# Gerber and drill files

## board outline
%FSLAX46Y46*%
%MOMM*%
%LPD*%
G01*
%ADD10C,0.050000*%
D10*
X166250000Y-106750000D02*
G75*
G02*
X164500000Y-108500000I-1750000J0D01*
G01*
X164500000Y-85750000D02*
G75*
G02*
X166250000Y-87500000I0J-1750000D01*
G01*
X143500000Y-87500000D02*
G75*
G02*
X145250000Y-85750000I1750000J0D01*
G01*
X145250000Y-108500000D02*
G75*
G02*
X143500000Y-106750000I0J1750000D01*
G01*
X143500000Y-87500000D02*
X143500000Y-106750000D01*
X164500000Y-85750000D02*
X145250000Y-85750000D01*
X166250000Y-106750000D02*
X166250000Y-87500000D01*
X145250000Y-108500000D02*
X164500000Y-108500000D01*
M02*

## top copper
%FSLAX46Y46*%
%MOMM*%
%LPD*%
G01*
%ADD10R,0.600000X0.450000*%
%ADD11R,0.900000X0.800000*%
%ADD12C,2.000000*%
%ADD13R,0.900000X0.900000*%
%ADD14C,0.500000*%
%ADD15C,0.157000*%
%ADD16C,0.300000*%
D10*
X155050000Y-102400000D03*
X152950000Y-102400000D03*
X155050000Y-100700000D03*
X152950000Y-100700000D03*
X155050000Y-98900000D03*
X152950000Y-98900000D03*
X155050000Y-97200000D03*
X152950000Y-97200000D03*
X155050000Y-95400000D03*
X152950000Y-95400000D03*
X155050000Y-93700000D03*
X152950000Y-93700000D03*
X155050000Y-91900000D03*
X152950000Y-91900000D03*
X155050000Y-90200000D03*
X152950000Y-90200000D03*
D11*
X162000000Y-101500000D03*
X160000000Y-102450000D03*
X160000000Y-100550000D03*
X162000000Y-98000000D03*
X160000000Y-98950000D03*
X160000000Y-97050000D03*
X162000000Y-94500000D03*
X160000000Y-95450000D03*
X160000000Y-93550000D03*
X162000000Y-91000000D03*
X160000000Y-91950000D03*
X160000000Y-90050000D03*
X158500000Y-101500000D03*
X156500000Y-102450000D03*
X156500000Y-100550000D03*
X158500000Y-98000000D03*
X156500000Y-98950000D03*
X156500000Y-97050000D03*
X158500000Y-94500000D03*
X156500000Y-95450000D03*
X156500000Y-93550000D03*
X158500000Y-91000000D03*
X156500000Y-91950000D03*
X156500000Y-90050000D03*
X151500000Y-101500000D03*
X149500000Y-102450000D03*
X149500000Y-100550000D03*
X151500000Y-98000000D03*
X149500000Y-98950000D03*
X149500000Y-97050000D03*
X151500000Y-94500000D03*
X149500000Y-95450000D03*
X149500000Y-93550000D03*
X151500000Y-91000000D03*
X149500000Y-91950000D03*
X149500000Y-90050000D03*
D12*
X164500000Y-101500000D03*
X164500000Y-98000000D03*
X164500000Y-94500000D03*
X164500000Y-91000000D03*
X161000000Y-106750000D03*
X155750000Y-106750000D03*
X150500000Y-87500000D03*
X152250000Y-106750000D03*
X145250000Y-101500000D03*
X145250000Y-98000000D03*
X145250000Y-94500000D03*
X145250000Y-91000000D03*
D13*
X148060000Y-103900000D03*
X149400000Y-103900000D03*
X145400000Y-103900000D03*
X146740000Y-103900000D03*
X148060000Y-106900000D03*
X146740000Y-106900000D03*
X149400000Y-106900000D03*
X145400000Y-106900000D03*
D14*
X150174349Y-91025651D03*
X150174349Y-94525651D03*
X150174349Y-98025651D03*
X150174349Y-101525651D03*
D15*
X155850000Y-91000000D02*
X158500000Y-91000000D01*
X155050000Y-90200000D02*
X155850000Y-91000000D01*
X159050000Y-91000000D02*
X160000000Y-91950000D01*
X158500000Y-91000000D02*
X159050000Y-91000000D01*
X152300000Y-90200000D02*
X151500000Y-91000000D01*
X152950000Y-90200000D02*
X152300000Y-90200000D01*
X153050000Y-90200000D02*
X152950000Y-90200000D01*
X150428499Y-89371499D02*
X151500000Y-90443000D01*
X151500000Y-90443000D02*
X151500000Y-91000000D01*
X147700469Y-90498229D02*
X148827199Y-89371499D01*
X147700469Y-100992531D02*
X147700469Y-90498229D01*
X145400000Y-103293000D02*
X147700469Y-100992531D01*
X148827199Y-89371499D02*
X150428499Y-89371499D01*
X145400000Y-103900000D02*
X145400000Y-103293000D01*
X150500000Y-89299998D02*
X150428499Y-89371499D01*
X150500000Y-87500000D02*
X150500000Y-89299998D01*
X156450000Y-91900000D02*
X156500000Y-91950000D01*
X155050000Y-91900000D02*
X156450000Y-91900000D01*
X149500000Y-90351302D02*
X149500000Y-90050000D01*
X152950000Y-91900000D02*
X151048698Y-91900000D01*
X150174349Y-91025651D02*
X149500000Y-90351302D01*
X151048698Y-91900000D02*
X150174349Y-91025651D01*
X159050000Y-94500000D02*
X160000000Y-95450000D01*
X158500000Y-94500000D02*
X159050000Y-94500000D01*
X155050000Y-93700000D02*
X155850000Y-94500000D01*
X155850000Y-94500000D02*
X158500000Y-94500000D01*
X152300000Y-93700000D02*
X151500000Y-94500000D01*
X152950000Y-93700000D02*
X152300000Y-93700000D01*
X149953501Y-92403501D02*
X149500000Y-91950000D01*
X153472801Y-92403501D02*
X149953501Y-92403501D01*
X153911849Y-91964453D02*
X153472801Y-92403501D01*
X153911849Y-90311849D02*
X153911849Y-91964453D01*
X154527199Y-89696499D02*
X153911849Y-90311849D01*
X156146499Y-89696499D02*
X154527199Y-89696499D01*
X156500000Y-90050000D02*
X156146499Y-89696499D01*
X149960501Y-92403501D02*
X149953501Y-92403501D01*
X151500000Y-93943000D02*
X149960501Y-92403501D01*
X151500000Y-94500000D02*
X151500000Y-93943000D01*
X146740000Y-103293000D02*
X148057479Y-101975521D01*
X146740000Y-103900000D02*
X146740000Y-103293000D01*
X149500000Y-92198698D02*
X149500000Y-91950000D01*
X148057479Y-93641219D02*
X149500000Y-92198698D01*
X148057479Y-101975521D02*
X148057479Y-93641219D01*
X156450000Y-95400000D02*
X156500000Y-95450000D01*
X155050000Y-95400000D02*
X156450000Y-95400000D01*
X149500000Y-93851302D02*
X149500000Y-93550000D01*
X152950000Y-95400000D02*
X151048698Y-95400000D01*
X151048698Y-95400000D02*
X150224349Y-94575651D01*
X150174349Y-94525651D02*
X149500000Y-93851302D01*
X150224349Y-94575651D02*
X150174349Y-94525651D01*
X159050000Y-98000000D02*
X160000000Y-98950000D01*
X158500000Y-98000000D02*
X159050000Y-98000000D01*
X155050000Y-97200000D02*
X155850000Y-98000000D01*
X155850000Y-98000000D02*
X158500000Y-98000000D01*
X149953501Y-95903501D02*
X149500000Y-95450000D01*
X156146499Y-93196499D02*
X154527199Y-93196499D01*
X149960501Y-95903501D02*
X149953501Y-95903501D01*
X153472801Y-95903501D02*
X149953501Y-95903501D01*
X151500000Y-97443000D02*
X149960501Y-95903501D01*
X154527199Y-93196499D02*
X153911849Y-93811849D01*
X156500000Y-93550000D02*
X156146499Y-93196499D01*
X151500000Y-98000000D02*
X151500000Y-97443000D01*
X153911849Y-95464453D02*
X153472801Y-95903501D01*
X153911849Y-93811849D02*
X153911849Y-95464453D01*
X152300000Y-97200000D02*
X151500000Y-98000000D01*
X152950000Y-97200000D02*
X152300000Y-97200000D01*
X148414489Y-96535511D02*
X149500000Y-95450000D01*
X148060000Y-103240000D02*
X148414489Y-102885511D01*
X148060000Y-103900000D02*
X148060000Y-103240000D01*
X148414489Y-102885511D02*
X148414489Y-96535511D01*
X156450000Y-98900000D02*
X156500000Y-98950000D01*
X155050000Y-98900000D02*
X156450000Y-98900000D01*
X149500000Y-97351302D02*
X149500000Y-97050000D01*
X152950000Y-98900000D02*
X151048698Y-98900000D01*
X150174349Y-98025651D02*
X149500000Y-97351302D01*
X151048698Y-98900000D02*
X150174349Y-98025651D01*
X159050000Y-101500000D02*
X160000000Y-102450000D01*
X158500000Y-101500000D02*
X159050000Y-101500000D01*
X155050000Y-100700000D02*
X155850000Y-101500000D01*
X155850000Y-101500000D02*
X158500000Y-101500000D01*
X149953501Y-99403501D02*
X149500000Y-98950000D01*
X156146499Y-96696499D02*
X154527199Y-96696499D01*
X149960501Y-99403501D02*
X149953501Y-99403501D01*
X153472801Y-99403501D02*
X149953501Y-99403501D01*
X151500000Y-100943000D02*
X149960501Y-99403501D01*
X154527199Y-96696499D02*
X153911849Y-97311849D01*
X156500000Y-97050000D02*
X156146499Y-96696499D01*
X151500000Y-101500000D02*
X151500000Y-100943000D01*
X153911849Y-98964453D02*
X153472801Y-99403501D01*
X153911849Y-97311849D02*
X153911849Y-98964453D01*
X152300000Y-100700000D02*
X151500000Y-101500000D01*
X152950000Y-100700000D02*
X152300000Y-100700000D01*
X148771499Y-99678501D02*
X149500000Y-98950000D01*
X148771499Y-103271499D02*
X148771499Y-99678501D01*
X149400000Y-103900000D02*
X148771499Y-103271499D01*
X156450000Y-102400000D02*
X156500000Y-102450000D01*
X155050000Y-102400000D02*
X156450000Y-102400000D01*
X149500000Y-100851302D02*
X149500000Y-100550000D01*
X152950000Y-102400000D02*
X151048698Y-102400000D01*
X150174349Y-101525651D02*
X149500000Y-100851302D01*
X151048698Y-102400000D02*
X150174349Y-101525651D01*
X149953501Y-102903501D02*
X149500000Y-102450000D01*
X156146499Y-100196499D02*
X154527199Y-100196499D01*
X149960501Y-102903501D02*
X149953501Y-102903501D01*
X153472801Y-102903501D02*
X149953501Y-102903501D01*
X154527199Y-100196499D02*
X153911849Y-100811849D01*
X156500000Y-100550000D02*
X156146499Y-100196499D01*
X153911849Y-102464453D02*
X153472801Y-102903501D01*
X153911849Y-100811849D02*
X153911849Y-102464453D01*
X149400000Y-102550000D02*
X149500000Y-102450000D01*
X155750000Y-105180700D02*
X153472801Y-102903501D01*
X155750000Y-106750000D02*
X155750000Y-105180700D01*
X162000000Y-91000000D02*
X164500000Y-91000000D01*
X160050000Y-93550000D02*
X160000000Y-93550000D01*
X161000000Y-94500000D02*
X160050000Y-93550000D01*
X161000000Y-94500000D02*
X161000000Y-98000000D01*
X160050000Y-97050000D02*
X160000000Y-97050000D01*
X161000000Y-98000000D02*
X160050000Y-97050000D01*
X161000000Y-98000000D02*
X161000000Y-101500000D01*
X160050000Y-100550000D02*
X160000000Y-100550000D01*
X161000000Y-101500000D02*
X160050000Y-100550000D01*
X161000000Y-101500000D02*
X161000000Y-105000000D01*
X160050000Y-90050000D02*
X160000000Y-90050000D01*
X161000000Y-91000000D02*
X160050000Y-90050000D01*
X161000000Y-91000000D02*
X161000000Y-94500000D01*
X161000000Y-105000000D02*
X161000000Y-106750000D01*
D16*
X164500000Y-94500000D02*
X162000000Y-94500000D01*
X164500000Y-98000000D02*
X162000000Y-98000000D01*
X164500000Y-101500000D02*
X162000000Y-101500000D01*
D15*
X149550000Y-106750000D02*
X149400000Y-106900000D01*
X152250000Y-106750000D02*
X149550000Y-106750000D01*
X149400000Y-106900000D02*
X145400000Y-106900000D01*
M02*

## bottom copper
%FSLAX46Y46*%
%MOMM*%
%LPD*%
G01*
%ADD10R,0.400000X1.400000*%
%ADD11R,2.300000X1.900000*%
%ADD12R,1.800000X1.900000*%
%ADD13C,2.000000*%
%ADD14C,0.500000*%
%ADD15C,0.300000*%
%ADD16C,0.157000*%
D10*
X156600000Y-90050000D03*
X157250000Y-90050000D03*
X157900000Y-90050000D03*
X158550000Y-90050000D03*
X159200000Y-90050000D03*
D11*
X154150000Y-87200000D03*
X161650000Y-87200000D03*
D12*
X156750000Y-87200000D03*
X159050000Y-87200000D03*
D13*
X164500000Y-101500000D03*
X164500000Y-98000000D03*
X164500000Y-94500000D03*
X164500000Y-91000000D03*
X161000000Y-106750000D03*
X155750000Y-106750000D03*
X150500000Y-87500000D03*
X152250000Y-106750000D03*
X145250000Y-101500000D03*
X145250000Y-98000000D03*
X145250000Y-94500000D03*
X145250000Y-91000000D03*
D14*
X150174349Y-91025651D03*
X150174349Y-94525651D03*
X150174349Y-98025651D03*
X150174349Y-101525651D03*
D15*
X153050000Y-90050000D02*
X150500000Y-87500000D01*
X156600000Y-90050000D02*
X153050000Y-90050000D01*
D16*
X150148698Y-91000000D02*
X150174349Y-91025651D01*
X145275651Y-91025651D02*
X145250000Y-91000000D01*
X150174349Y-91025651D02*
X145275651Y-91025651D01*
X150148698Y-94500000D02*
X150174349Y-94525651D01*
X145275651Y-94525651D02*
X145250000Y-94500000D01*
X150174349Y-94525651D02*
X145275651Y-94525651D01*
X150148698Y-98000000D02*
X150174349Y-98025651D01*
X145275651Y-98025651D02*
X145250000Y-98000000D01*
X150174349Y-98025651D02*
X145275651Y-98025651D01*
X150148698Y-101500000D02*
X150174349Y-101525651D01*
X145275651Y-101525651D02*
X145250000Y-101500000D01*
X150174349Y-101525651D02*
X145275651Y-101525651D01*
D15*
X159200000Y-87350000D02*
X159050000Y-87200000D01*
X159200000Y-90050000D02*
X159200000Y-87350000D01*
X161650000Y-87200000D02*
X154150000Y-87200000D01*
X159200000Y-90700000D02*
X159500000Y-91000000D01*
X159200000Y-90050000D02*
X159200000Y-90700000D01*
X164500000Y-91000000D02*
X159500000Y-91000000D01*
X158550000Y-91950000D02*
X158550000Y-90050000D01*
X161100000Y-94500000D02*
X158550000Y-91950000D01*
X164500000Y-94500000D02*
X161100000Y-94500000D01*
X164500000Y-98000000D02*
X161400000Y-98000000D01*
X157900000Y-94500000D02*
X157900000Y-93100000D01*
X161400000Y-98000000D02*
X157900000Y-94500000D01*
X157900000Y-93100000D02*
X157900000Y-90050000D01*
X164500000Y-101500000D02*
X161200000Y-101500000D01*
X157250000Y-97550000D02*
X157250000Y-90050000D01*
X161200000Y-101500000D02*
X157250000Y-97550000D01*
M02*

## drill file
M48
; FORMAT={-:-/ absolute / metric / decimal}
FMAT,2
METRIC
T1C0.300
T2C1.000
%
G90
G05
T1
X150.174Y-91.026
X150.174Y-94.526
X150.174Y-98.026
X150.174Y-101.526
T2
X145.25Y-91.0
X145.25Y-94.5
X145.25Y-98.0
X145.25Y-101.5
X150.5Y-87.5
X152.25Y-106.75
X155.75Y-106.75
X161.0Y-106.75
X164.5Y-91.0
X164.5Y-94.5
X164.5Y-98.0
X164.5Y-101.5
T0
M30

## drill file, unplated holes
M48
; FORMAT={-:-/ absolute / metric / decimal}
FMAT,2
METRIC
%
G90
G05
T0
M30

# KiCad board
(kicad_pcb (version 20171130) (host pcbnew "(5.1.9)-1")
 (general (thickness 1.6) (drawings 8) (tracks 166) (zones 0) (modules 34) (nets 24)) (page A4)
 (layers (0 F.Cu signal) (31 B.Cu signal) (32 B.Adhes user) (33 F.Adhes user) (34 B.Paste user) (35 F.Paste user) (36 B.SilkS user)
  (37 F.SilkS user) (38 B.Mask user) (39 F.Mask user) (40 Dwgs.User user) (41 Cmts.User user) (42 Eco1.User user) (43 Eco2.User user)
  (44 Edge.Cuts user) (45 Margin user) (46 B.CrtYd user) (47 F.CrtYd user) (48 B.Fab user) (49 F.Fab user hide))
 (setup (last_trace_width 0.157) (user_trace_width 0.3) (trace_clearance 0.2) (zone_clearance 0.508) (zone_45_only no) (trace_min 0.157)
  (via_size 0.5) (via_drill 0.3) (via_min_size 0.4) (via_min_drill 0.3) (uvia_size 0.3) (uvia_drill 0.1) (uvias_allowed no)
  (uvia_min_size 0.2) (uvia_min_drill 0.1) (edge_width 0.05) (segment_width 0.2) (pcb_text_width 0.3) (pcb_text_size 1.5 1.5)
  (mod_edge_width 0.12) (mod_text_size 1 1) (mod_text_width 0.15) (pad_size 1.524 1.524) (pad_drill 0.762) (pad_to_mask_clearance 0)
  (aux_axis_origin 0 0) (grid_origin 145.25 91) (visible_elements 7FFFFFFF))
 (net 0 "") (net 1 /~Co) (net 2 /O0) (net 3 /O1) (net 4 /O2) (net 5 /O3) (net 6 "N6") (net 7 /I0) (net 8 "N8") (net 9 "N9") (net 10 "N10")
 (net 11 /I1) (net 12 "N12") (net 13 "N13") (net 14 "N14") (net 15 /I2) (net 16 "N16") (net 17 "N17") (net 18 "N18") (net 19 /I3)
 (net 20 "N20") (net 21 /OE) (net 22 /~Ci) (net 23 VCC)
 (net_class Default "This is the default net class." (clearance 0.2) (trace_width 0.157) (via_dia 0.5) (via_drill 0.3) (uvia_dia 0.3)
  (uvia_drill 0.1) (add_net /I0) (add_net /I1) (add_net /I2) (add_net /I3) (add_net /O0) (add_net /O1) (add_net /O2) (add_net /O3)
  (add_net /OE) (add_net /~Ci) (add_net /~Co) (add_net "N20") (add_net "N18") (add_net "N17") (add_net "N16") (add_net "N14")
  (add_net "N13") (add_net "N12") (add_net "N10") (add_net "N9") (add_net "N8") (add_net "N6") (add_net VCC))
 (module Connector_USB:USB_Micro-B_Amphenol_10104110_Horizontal (layer B.Cu) (at 157.9 88.5)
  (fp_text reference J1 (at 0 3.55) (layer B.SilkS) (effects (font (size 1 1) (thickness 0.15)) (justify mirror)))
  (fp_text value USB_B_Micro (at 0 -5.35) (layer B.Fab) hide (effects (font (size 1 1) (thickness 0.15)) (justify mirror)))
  (pad 1 smd rect (at -1.3 1.55) (size 0.4 1.4) (layers B.Cu B.Paste B.Mask) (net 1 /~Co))
  (pad 2 smd rect (at -0.65 1.55) (size 0.4 1.4) (layers B.Cu B.Paste B.Mask) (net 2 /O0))
  (pad 3 smd rect (at 0 1.55) (size 0.4 1.4) (layers B.Cu B.Paste B.Mask) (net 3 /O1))
  (pad 4 smd rect (at 0.65 1.55) (size 0.4 1.4) (layers B.Cu B.Paste B.Mask) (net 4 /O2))
  (pad 5 smd rect (at 1.3 1.55) (size 0.4 1.4) (layers B.Cu B.Paste B.Mask) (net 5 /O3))
  (pad 6 smd rect (at -3.75 -1.3) (size 2.3 1.9) (layers B.Cu B.Paste B.Mask) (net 5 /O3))
  (pad 6 smd rect (at 3.75 -1.3) (size 2.3 1.9) (layers B.Cu B.Paste B.Mask) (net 5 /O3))
  (pad 6 smd rect (at -1.15 -1.3) (size 1.8 1.9) (layers B.Cu B.Paste B.Mask) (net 5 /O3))
  (pad 6 smd rect (at 1.15 -1.3) (size 1.8 1.9) (layers B.Cu B.Paste B.Mask) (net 5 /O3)))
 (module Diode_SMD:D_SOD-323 (layer F.Cu) (at 154 102.4)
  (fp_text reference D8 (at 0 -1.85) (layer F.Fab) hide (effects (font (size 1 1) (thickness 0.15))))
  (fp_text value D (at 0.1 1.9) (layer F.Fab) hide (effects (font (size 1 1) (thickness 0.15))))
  (pad 2 smd rect (at 1.05 0) (size 0.6 0.45) (layers F.Cu F.Paste F.Mask) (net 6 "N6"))
  (pad 1 smd rect (at -1.05 0) (size 0.6 0.45) (layers F.Cu F.Paste F.Mask) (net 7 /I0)))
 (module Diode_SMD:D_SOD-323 (layer F.Cu) (at 154 100.7)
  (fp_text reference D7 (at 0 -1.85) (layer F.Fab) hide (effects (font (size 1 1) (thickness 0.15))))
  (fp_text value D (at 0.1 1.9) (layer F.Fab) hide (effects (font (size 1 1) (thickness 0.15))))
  (pad 2 smd rect (at 1.05 0) (size 0.6 0.45) (layers F.Cu F.Paste F.Mask) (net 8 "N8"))
  (pad 1 smd rect (at -1.05 0) (size 0.6 0.45) (layers F.Cu F.Paste F.Mask) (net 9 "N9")))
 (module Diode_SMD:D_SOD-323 (layer F.Cu) (at 154 98.9)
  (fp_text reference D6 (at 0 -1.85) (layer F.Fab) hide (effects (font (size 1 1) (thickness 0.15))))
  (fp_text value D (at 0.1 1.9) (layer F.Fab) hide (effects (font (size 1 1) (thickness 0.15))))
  (pad 2 smd rect (at 1.05 0) (size 0.6 0.45) (layers F.Cu F.Paste F.Mask) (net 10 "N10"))
  (pad 1 smd rect (at -1.05 0) (size 0.6 0.45) (layers F.Cu F.Paste F.Mask) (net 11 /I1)))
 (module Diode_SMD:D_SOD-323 (layer F.Cu) (at 154 97.2)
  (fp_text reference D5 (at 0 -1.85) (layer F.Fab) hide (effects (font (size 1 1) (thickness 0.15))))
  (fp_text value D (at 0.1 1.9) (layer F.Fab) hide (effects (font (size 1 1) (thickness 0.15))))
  (pad 2 smd rect (at 1.05 0) (size 0.6 0.45) (layers F.Cu F.Paste F.Mask) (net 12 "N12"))
  (pad 1 smd rect (at -1.05 0) (size 0.6 0.45) (layers F.Cu F.Paste F.Mask) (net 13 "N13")))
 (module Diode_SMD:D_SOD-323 (layer F.Cu) (at 154 95.4)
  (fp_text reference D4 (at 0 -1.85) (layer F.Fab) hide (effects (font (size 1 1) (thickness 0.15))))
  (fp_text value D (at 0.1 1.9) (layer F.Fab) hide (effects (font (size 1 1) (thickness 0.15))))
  (pad 2 smd rect (at 1.05 0) (size 0.6 0.45) (layers F.Cu F.Paste F.Mask) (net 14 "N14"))
  (pad 1 smd rect (at -1.05 0) (size 0.6 0.45) (layers F.Cu F.Paste F.Mask) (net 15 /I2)))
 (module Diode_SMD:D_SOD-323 (layer F.Cu) (at 154 93.7)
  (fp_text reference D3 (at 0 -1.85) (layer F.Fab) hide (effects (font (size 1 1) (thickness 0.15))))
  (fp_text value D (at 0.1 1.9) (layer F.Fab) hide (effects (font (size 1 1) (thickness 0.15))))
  (pad 2 smd rect (at 1.05 0) (size 0.6 0.45) (layers F.Cu F.Paste F.Mask) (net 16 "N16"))
  (pad 1 smd rect (at -1.05 0) (size 0.6 0.45) (layers F.Cu F.Paste F.Mask) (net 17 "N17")))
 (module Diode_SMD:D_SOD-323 (layer F.Cu) (at 154 91.9)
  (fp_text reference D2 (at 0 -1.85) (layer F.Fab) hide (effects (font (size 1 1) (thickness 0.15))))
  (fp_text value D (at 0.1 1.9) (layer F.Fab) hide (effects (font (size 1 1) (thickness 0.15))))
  (pad 2 smd rect (at 1.05 0) (size 0.6 0.45) (layers F.Cu F.Paste F.Mask) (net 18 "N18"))
  (pad 1 smd rect (at -1.05 0) (size 0.6 0.45) (layers F.Cu F.Paste F.Mask) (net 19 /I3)))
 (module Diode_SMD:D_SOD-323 (layer F.Cu) (at 154 90.2)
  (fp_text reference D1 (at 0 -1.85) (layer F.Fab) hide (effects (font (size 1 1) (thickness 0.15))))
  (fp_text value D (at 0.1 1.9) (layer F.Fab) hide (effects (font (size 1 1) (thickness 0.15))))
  (pad 2 smd rect (at 1.05 0) (size 0.6 0.45) (layers F.Cu F.Paste F.Mask) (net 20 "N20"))
  (pad 1 smd rect (at -1.05 0) (size 0.6 0.45) (layers F.Cu F.Paste F.Mask) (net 1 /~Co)))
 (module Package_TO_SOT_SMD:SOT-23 (layer F.Cu) (at 161 101.5)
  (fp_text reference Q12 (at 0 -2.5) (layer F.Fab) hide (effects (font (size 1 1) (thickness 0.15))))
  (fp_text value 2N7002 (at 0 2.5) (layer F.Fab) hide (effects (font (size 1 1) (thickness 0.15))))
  (pad 3 smd rect (at 1 0) (size 0.9 0.8) (layers F.Cu F.Paste F.Mask) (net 2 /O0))
  (pad 2 smd rect (at -1 0.95) (size 0.9 0.8) (layers F.Cu F.Paste F.Mask) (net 8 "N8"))
  (pad 1 smd rect (at -1 -0.95) (size 0.9 0.8) (layers F.Cu F.Paste F.Mask) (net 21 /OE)))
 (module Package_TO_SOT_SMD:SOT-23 (layer F.Cu) (at 161 98)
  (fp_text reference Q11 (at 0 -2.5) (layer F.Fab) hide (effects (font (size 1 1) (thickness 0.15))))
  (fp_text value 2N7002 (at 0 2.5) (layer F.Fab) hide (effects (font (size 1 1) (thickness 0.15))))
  (pad 3 smd rect (at 1 0) (size 0.9 0.8) (layers F.Cu F.Paste F.Mask) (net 3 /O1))
  (pad 2 smd rect (at -1 0.95) (size 0.9 0.8) (layers F.Cu F.Paste F.Mask) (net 12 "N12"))
  (pad 1 smd rect (at -1 -0.95) (size 0.9 0.8) (layers F.Cu F.Paste F.Mask) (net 21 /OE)))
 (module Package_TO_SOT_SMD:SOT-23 (layer F.Cu) (at 161 94.5)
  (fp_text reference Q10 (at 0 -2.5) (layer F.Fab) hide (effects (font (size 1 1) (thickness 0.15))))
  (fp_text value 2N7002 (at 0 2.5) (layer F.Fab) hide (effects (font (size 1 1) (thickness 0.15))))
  (pad 3 smd rect (at 1 0) (size 0.9 0.8) (layers F.Cu F.Paste F.Mask) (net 4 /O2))
  (pad 2 smd rect (at -1 0.95) (size 0.9 0.8) (layers F.Cu F.Paste F.Mask) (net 16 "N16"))
  (pad 1 smd rect (at -1 -0.95) (size 0.9 0.8) (layers F.Cu F.Paste F.Mask) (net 21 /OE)))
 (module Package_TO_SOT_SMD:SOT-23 (layer F.Cu) (at 161 91)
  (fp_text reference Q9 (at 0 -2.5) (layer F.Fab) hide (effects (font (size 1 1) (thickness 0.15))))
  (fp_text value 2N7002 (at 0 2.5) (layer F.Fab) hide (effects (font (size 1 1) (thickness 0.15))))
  (pad 3 smd rect (at 1 0) (size 0.9 0.8) (layers F.Cu F.Paste F.Mask) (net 5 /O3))
  (pad 2 smd rect (at -1 0.95) (size 0.9 0.8) (layers F.Cu F.Paste F.Mask) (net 20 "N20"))
  (pad 1 smd rect (at -1 -0.95) (size 0.9 0.8) (layers F.Cu F.Paste F.Mask) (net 21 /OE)))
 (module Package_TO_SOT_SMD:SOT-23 (layer F.Cu) (at 157.5 101.5)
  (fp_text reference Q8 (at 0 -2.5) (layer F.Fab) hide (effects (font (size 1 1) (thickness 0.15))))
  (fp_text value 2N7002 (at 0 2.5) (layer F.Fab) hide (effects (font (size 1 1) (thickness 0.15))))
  (pad 3 smd rect (at 1 0) (size 0.9 0.8) (layers F.Cu F.Paste F.Mask) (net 8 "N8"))
  (pad 2 smd rect (at -1 0.95) (size 0.9 0.8) (layers F.Cu F.Paste F.Mask) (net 6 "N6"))
  (pad 1 smd rect (at -1 -0.95) (size 0.9 0.8) (layers F.Cu F.Paste F.Mask) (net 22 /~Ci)))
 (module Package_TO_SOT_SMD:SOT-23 (layer F.Cu) (at 157.5 98)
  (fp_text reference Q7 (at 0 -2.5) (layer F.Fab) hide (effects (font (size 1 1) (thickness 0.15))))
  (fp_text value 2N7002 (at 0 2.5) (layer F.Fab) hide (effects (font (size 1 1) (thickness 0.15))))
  (pad 3 smd rect (at 1 0) (size 0.9 0.8) (layers F.Cu F.Paste F.Mask) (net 12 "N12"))
  (pad 2 smd rect (at -1 0.95) (size 0.9 0.8) (layers F.Cu F.Paste F.Mask) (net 10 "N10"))
  (pad 1 smd rect (at -1 -0.95) (size 0.9 0.8) (layers F.Cu F.Paste F.Mask) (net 9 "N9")))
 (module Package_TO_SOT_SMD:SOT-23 (layer F.Cu) (at 157.5 94.5)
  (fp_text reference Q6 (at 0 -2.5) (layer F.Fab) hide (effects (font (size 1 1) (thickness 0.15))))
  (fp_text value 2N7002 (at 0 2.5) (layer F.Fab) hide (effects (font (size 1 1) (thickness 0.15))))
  (pad 3 smd rect (at 1 0) (size 0.9 0.8) (layers F.Cu F.Paste F.Mask) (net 16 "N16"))
  (pad 2 smd rect (at -1 0.95) (size 0.9 0.8) (layers F.Cu F.Paste F.Mask) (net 14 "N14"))
  (pad 1 smd rect (at -1 -0.95) (size 0.9 0.8) (layers F.Cu F.Paste F.Mask) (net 13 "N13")))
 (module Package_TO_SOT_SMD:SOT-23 (layer F.Cu) (at 157.5 91)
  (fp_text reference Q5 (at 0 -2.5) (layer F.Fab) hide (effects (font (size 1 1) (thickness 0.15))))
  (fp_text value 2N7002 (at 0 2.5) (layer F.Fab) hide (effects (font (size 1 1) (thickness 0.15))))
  (pad 3 smd rect (at 1 0) (size 0.9 0.8) (layers F.Cu F.Paste F.Mask) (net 20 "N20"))
  (pad 2 smd rect (at -1 0.95) (size 0.9 0.8) (layers F.Cu F.Paste F.Mask) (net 18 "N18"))
  (pad 1 smd rect (at -1 -0.95) (size 0.9 0.8) (layers F.Cu F.Paste F.Mask) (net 17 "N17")))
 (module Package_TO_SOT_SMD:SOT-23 (layer F.Cu) (at 150.5 101.5)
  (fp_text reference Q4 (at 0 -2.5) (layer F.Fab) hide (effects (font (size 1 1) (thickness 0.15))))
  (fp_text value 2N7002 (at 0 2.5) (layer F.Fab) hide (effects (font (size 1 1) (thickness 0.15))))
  (pad 3 smd rect (at 1 0) (size 0.9 0.8) (layers F.Cu F.Paste F.Mask) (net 9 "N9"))
  (pad 2 smd rect (at -1 0.95) (size 0.9 0.8) (layers F.Cu F.Paste F.Mask) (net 22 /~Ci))
  (pad 1 smd rect (at -1 -0.95) (size 0.9 0.8) (layers F.Cu F.Paste F.Mask) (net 7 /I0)))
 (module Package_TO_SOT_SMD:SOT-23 (layer F.Cu) (at 150.5 98)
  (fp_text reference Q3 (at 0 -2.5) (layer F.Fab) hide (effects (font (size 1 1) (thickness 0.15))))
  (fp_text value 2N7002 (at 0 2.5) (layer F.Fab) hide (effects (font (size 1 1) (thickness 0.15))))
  (pad 3 smd rect (at 1 0) (size 0.9 0.8) (layers F.Cu F.Paste F.Mask) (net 13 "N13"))
  (pad 2 smd rect (at -1 0.95) (size 0.9 0.8) (layers F.Cu F.Paste F.Mask) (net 9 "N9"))
  (pad 1 smd rect (at -1 -0.95) (size 0.9 0.8) (layers F.Cu F.Paste F.Mask) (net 11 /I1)))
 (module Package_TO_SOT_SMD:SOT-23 (layer F.Cu) (at 150.5 94.5)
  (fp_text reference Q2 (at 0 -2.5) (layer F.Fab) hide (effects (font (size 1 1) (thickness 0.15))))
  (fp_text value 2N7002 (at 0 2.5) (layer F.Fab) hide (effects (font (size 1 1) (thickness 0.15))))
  (pad 3 smd rect (at 1 0) (size 0.9 0.8) (layers F.Cu F.Paste F.Mask) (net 17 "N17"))
  (pad 2 smd rect (at -1 0.95) (size 0.9 0.8) (layers F.Cu F.Paste F.Mask) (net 13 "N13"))
  (pad 1 smd rect (at -1 -0.95) (size 0.9 0.8) (layers F.Cu F.Paste F.Mask) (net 15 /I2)))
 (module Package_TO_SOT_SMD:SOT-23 (layer F.Cu) (at 150.5 91)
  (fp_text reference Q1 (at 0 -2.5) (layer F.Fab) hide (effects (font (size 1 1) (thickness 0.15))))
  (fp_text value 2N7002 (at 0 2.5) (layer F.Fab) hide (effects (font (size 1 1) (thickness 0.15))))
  (pad 3 smd rect (at 1 0) (size 0.9 0.8) (layers F.Cu F.Paste F.Mask) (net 1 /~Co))
  (pad 2 smd rect (at -1 0.95) (size 0.9 0.8) (layers F.Cu F.Paste F.Mask) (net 17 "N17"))
  (pad 1 smd rect (at -1 -0.95) (size 0.9 0.8) (layers F.Cu F.Paste F.Mask) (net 19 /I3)))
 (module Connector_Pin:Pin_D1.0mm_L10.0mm (layer F.Cu) (at 164.5 101.5)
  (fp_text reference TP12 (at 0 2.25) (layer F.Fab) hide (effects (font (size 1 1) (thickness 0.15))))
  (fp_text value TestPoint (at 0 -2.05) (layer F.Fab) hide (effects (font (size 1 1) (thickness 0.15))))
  (pad 1 thru_hole circle (at 0 0) (size 2 2) (drill 1) (layers *.Cu *.Mask) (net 2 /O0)))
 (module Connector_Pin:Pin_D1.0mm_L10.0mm (layer F.Cu) (at 164.5 98)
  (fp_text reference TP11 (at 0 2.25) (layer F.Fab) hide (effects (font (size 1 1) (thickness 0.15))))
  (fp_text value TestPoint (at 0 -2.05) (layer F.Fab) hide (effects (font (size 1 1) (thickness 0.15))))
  (pad 1 thru_hole circle (at 0 0) (size 2 2) (drill 1) (layers *.Cu *.Mask) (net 3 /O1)))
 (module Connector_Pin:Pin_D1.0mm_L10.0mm (layer F.Cu) (at 164.5 94.5)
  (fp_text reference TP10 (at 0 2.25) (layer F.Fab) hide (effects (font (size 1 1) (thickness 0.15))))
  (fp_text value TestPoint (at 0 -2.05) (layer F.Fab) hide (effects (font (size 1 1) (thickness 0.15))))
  (pad 1 thru_hole circle (at 0 0) (size 2 2) (drill 1) (layers *.Cu *.Mask) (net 4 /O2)))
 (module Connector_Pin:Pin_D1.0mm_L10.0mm (layer F.Cu) (at 164.5 91)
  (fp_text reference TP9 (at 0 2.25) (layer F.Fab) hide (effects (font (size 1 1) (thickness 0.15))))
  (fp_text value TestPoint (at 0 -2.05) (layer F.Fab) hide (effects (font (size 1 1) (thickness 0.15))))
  (pad 1 thru_hole circle (at 0 0) (size 2 2) (drill 1) (layers *.Cu *.Mask) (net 5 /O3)))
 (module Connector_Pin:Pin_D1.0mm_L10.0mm (layer F.Cu) (at 161 106.75)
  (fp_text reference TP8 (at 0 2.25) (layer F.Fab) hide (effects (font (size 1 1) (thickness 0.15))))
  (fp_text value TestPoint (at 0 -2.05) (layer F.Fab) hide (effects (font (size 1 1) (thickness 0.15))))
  (pad 1 thru_hole circle (at 0 0) (size 2 2) (drill 1) (layers *.Cu *.Mask) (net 21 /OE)))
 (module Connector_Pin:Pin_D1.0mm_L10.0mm (layer F.Cu) (at 155.75 106.75)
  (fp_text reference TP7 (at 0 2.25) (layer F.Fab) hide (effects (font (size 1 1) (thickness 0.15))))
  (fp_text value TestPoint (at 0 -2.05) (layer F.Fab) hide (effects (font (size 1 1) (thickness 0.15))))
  (pad 1 thru_hole circle (at 0 0) (size 2 2) (drill 1) (layers *.Cu *.Mask) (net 22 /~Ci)))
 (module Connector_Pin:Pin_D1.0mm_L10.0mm (layer F.Cu) (at 150.5 87.5)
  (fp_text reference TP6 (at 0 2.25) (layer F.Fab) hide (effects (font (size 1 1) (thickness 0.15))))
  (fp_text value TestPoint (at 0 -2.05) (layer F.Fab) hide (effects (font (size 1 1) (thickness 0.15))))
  (pad 1 thru_hole circle (at 0 0) (size 2 2) (drill 1) (layers *.Cu *.Mask) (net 1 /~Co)))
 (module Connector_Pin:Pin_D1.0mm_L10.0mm (layer F.Cu) (at 152.25 106.75)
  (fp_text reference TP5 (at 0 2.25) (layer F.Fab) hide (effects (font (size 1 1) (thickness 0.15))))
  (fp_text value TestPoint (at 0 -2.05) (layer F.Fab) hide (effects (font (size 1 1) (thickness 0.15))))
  (pad 1 thru_hole circle (at 0 0) (size 2 2) (drill 1) (layers *.Cu *.Mask) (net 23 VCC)))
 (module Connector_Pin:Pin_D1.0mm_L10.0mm (layer F.Cu) (at 145.25 101.5)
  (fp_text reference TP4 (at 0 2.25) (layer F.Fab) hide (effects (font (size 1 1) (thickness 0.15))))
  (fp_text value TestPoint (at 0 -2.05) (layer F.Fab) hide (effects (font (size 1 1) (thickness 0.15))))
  (pad 1 thru_hole circle (at 0 0) (size 2 2) (drill 1) (layers *.Cu *.Mask) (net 7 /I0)))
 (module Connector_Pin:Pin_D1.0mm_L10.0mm (layer F.Cu) (at 145.25 98)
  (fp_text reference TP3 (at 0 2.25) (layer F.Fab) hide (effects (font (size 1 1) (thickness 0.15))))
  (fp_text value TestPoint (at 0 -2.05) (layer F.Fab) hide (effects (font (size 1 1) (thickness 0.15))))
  (pad 1 thru_hole circle (at 0 0) (size 2 2) (drill 1) (layers *.Cu *.Mask) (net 11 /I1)))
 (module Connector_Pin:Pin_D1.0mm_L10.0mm (layer F.Cu) (at 145.25 94.5)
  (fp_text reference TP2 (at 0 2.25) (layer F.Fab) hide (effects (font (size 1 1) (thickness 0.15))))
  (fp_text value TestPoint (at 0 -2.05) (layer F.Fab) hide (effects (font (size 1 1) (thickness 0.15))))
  (pad 1 thru_hole circle (at 0 0) (size 2 2) (drill 1) (layers *.Cu *.Mask) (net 15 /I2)))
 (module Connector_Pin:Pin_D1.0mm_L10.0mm (layer F.Cu) (at 145.25 91)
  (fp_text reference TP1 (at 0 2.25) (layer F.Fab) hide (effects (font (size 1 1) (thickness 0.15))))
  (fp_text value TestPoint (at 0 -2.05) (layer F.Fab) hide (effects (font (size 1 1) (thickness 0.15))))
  (pad 1 thru_hole circle (at 0 0) (size 2 2) (drill 1) (layers *.Cu *.Mask) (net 19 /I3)))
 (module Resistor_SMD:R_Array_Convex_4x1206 (layer F.Cu) (at 147.4 105.4 90)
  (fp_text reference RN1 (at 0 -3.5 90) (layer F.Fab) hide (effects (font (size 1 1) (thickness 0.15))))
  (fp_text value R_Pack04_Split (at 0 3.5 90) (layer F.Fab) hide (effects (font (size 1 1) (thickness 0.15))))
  (pad 6 smd rect (at 1.5 0.66 90) (size 0.9 0.9) (layers F.Cu F.Paste F.Mask) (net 13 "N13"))
  (pad 5 smd rect (at 1.5 2 90) (size 0.9 0.9) (layers F.Cu F.Paste F.Mask) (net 9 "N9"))
  (pad 8 smd rect (at 1.5 -2 90) (size 0.9 0.9) (layers F.Cu F.Paste F.Mask) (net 1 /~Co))
  (pad 7 smd rect (at 1.5 -0.66 90) (size 0.9 0.9) (layers F.Cu F.Paste F.Mask) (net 17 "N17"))
  (pad 3 smd rect (at -1.5 0.66 90) (size 0.9 0.9) (layers F.Cu F.Paste F.Mask) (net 23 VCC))
  (pad 2 smd rect (at -1.5 -0.66 90) (size 0.9 0.9) (layers F.Cu F.Paste F.Mask) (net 23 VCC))
  (pad 4 smd rect (at -1.5 2 90) (size 0.9 0.9) (layers F.Cu F.Paste F.Mask) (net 23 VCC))
  (pad 1 smd rect (at -1.5 -2 90) (size 0.9 0.9) (layers F.Cu F.Paste F.Mask) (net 23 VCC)))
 (gr_arc (start 164.5 106.75) (end 164.5 108.5) (angle -90) (layer Edge.Cuts) (width 0.05))
 (gr_arc (start 164.5 87.5) (end 166.25 87.5) (angle -90) (layer Edge.Cuts) (width 0.05))
 (gr_arc (start 145.25 87.5) (end 145.25 85.75) (angle -90) (layer Edge.Cuts) (width 0.05))
 (gr_arc (start 145.25 106.75) (end 143.5 106.75) (angle -90) (layer Edge.Cuts) (width 0.05))
 (gr_line (start 143.5 87.5) (end 143.5 106.75) (layer Edge.Cuts) (width 0.05))
 (gr_line (start 164.5 85.75) (end 145.25 85.75) (layer Edge.Cuts) (width 0.05))
 (gr_line (start 166.25 106.75) (end 166.25 87.5) (layer Edge.Cuts) (width 0.05))
 (gr_line (start 145.25 108.5) (end 164.5 108.5) (layer Edge.Cuts) (width 0.05))
 (segment (start 155.85 91) (end 158.5 91) (width 0.157) (layer F.Cu) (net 20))
 (segment (start 155.05 90.2) (end 155.85 91) (width 0.157) (layer F.Cu) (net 20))
 (segment (start 159.05 91) (end 160 91.95) (width 0.157) (layer F.Cu) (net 20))
 (segment (start 158.5 91) (end 159.05 91) (width 0.157) (layer F.Cu) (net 20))
 (segment (start 152.3 90.2) (end 151.5 91) (width 0.157) (layer F.Cu) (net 1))
 (segment (start 152.95 90.2) (end 152.3 90.2) (width 0.157) (layer F.Cu) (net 1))
 (segment (start 153.05 90.2) (end 152.95 90.2) (width 0.157) (layer F.Cu) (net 1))
 (segment (start 150.428499 89.371499) (end 151.5 90.443) (width 0.157) (layer F.Cu) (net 1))
 (segment (start 151.5 90.443) (end 151.5 91) (width 0.157) (layer F.Cu) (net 1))
 (segment (start 147.700469 90.498229) (end 148.827199 89.371499) (width 0.157) (layer F.Cu) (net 1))
 (segment (start 147.700469 100.992531) (end 147.700469 90.498229) (width 0.157) (layer F.Cu) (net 1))
 (segment (start 145.4 103.293) (end 147.700469 100.992531) (width 0.157) (layer F.Cu) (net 1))
 (segment (start 148.827199 89.371499) (end 150.428499 89.371499) (width 0.157) (layer F.Cu) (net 1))
 (segment (start 145.4 103.9) (end 145.4 103.293) (width 0.157) (layer F.Cu) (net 1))
 (segment (start 150.5 89.299998) (end 150.428499 89.371499) (width 0.157) (layer F.Cu) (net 1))
 (segment (start 150.5 87.5) (end 150.5 89.299998) (width 0.157) (layer F.Cu) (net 1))
 (segment (start 153.05 90.05) (end 150.5 87.5) (width 0.3) (layer B.Cu) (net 1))
 (segment (start 156.6 90.05) (end 153.05 90.05) (width 0.3) (layer B.Cu) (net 1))
 (segment (start 156.45 91.9) (end 156.5 91.95) (width 0.157) (layer F.Cu) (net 18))
 (segment (start 155.05 91.9) (end 156.45 91.9) (width 0.157) (layer F.Cu) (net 18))
 (segment (start 149.5 90.351302) (end 149.5 90.05) (width 0.157) (layer F.Cu) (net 19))
 (segment (start 152.95 91.9) (end 151.048698 91.9) (width 0.157) (layer F.Cu) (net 19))
 (via (at 150.174349 91.025651) (size 0.5) (drill 0.3) (layers F.Cu B.Cu) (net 19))
 (segment (start 150.148698 91) (end 150.174349 91.025651) (width 0.157) (layer B.Cu) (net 19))
 (segment (start 150.174349 91.025651) (end 149.5 90.351302) (width 0.157) (layer F.Cu) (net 19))
 (segment (start 151.048698 91.9) (end 150.174349 91.025651) (width 0.157) (layer F.Cu) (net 19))
 (segment (start 145.275651 91.025651) (end 145.25 91) (width 0.157) (layer B.Cu) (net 19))
 (segment (start 150.174349 91.025651) (end 145.275651 91.025651) (width 0.157) (layer B.Cu) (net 19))
 (segment (start 159.05 94.5) (end 160 95.45) (width 0.157) (layer F.Cu) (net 16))
 (segment (start 158.5 94.5) (end 159.05 94.5) (width 0.157) (layer F.Cu) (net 16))
 (segment (start 155.05 93.7) (end 155.85 94.5) (width 0.157) (layer F.Cu) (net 16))
 (segment (start 155.85 94.5) (end 158.5 94.5) (width 0.157) (layer F.Cu) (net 16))
 (segment (start 152.3 93.7) (end 151.5 94.5) (width 0.157) (layer F.Cu) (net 17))
 (segment (start 152.95 93.7) (end 152.3 93.7) (width 0.157) (layer F.Cu) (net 17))
 (segment (start 149.953501 92.403501) (end 149.5 91.95) (width 0.157) (layer F.Cu) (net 17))
 (segment (start 153.472801 92.403501) (end 149.953501 92.403501) (width 0.157) (layer F.Cu) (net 17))
 (segment (start 153.911849 91.964453) (end 153.472801 92.403501) (width 0.157) (layer F.Cu) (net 17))
 (segment (start 153.911849 90.311849) (end 153.911849 91.964453) (width 0.157) (layer F.Cu) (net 17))
 (segment (start 154.527199 89.696499) (end 153.911849 90.311849) (width 0.157) (layer F.Cu) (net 17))
 (segment (start 156.146499 89.696499) (end 154.527199 89.696499) (width 0.157) (layer F.Cu) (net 17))
 (segment (start 156.5 90.05) (end 156.146499 89.696499) (width 0.157) (layer F.Cu) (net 17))
 (segment (start 149.960501 92.403501) (end 149.953501 92.403501) (width 0.157) (layer F.Cu) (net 17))
 (segment (start 151.5 93.943) (end 149.960501 92.403501) (width 0.157) (layer F.Cu) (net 17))
 (segment (start 151.5 94.5) (end 151.5 93.943) (width 0.157) (layer F.Cu) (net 17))
 (segment (start 146.74 103.293) (end 148.057479 101.975521) (width 0.157) (layer F.Cu) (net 17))
 (segment (start 146.74 103.9) (end 146.74 103.293) (width 0.157) (layer F.Cu) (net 17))
 (segment (start 149.5 92.198698) (end 149.5 91.95) (width 0.157) (layer F.Cu) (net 17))
 (segment (start 148.057479 93.641219) (end 149.5 92.198698) (width 0.157) (layer F.Cu) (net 17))
 (segment (start 148.057479 101.975521) (end 148.057479 93.641219) (width 0.157) (layer F.Cu) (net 17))
 (segment (start 156.45 95.4) (end 156.5 95.45) (width 0.157) (layer F.Cu) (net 14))
 (segment (start 155.05 95.4) (end 156.45 95.4) (width 0.157) (layer F.Cu) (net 14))
 (segment (start 149.5 93.851302) (end 149.5 93.55) (width 0.157) (layer F.Cu) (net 15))
 (segment (start 152.95 95.4) (end 151.048698 95.4) (width 0.157) (layer F.Cu) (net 15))
 (segment (start 151.048698 95.4) (end 150.224349 94.575651) (width 0.157) (layer F.Cu) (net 15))
 (via (at 150.174349 94.525651) (size 0.5) (drill 0.3) (layers F.Cu B.Cu) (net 15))
 (segment (start 150.174349 94.525651) (end 149.5 93.851302) (width 0.157) (layer F.Cu) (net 15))
 (segment (start 150.148698 94.5) (end 150.174349 94.525651) (width 0.157) (layer B.Cu) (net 15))
 (segment (start 150.224349 94.575651) (end 150.174349 94.525651) (width 0.157) (layer F.Cu) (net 15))
 (segment (start 145.275651 94.525651) (end 145.25 94.5) (width 0.157) (layer B.Cu) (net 15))
 (segment (start 150.174349 94.525651) (end 145.275651 94.525651) (width 0.157) (layer B.Cu) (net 15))
 (segment (start 159.05 98) (end 160 98.95) (width 0.157) (layer F.Cu) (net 12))
 (segment (start 158.5 98) (end 159.05 98) (width 0.157) (layer F.Cu) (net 12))
 (segment (start 155.05 97.2) (end 155.85 98) (width 0.157) (layer F.Cu) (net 12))
 (segment (start 155.85 98) (end 158.5 98) (width 0.157) (layer F.Cu) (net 12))
 (segment (start 149.953501 95.903501) (end 149.5 95.45) (width 0.157) (layer F.Cu) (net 13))
 (segment (start 156.146499 93.196499) (end 154.527199 93.196499) (width 0.157) (layer F.Cu) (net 13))
 (segment (start 149.960501 95.903501) (end 149.953501 95.903501) (width 0.157) (layer F.Cu) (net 13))
 (segment (start 153.472801 95.903501) (end 149.953501 95.903501) (width 0.157) (layer F.Cu) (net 13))
 (segment (start 151.5 97.443) (end 149.960501 95.903501) (width 0.157) (layer F.Cu) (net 13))
 (segment (start 154.527199 93.196499) (end 153.911849 93.811849) (width 0.157) (layer F.Cu) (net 13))
 (segment (start 156.5 93.55) (end 156.146499 93.196499) (width 0.157) (layer F.Cu) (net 13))
 (segment (start 151.5 98) (end 151.5 97.443) (width 0.157) (layer F.Cu) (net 13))
 (segment (start 153.911849 95.464453) (end 153.472801 95.903501) (width 0.157) (layer F.Cu) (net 13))
 (segment (start 153.911849 93.811849) (end 153.911849 95.464453) (width 0.157) (layer F.Cu) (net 13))
 (segment (start 152.3 97.2) (end 151.5 98) (width 0.157) (layer F.Cu) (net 13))
 (segment (start 152.95 97.2) (end 152.3 97.2) (width 0.157) (layer F.Cu) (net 13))
 (segment (start 148.414489 96.535511) (end 149.5 95.45) (width 0.157) (layer F.Cu) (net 13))
 (segment (start 148.06 103.24) (end 148.414489 102.885511) (width 0.157) (layer F.Cu) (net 13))
 (segment (start 148.06 103.9) (end 148.06 103.24) (width 0.157) (layer F.Cu) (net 13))
 (segment (start 148.414489 102.885511) (end 148.414489 96.535511) (width 0.157) (layer F.Cu) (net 13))
 (segment (start 156.45 98.9) (end 156.5 98.95) (width 0.157) (layer F.Cu) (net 10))
 (segment (start 155.05 98.9) (end 156.45 98.9) (width 0.157) (layer F.Cu) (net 10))
 (segment (start 149.5 97.351302) (end 149.5 97.05) (width 0.157) (layer F.Cu) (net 11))
 (segment (start 152.95 98.9) (end 151.048698 98.9) (width 0.157) (layer F.Cu) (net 11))
 (via (at 150.174349 98.025651) (size 0.5) (drill 0.3) (layers F.Cu B.Cu) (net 11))
 (segment (start 150.148698 98) (end 150.174349 98.025651) (width 0.157) (layer B.Cu) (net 11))
 (segment (start 150.174349 98.025651) (end 149.5 97.351302) (width 0.157) (layer F.Cu) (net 11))
 (segment (start 151.048698 98.9) (end 150.174349 98.025651) (width 0.157) (layer F.Cu) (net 11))
 (segment (start 145.275651 98.025651) (end 145.25 98) (width 0.157) (layer B.Cu) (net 11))
 (segment (start 150.174349 98.025651) (end 145.275651 98.025651) (width 0.157) (layer B.Cu) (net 11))
 (segment (start 159.05 101.5) (end 160 102.45) (width 0.157) (layer F.Cu) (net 8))
 (segment (start 158.5 101.5) (end 159.05 101.5) (width 0.157) (layer F.Cu) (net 8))
 (segment (start 155.05 100.7) (end 155.85 101.5) (width 0.157) (layer F.Cu) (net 8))
 (segment (start 155.85 101.5) (end 158.5 101.5) (width 0.157) (layer F.Cu) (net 8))
 (segment (start 149.953501 99.403501) (end 149.5 98.95) (width 0.157) (layer F.Cu) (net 9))
 (segment (start 156.146499 96.696499) (end 154.527199 96.696499) (width 0.157) (layer F.Cu) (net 9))
 (segment (start 149.960501 99.403501) (end 149.953501 99.403501) (width 0.157) (layer F.Cu) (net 9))
 (segment (start 153.472801 99.403501) (end 149.953501 99.403501) (width 0.157) (layer F.Cu) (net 9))
 (segment (start 151.5 100.943) (end 149.960501 99.403501) (width 0.157) (layer F.Cu) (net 9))
 (segment (start 154.527199 96.696499) (end 153.911849 97.311849) (width 0.157) (layer F.Cu) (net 9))
 (segment (start 156.5 97.05) (end 156.146499 96.696499) (width 0.157) (layer F.Cu) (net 9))
 (segment (start 151.5 101.5) (end 151.5 100.943) (width 0.157) (layer F.Cu) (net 9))
 (segment (start 153.911849 98.964453) (end 153.472801 99.403501) (width 0.157) (layer F.Cu) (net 9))
 (segment (start 153.911849 97.311849) (end 153.911849 98.964453) (width 0.157) (layer F.Cu) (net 9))
 (segment (start 152.3 100.7) (end 151.5 101.5) (width 0.157) (layer F.Cu) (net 9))
 (segment (start 152.95 100.7) (end 152.3 100.7) (width 0.157) (layer F.Cu) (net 9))
 (segment (start 148.771499 99.678501) (end 149.5 98.95) (width 0.157) (layer F.Cu) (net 9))
 (segment (start 148.771499 103.271499) (end 148.771499 99.678501) (width 0.157) (layer F.Cu) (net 9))
 (segment (start 149.4 103.9) (end 148.771499 103.271499) (width 0.157) (layer F.Cu) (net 9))
 (segment (start 156.45 102.4) (end 156.5 102.45) (width 0.157) (layer F.Cu) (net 6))
 (segment (start 155.05 102.4) (end 156.45 102.4) (width 0.157) (layer F.Cu) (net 6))
 (segment (start 149.5 100.851302) (end 149.5 100.55) (width 0.157) (layer F.Cu) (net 7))
 (segment (start 152.95 102.4) (end 151.048698 102.4) (width 0.157) (layer F.Cu) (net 7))
 (via (at 150.174349 101.525651) (size 0.5) (drill 0.3) (layers F.Cu B.Cu) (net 7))
 (segment (start 150.174349 101.525651) (end 149.5 100.851302) (width 0.157) (layer F.Cu) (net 7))
 (segment (start 151.048698 102.4) (end 150.174349 101.525651) (width 0.157) (layer F.Cu) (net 7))
 (segment (start 150.148698 101.5) (end 150.174349 101.525651) (width 0.157) (layer B.Cu) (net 7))
 (segment (start 145.275651 101.525651) (end 145.25 101.5) (width 0.157) (layer B.Cu) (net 7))
 (segment (start 150.174349 101.525651) (end 145.275651 101.525651) (width 0.157) (layer B.Cu) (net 7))
 (segment (start 149.953501 102.903501) (end 149.5 102.45) (width 0.157) (layer F.Cu) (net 22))
 (segment (start 156.146499 100.196499) (end 154.527199 100.196499) (width 0.157) (layer F.Cu) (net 22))
 (segment (start 149.960501 102.903501) (end 149.953501 102.903501) (width 0.157) (layer F.Cu) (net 22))
 (segment (start 153.472801 102.903501) (end 149.953501 102.903501) (width 0.157) (layer F.Cu) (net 22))
 (segment (start 154.527199 100.196499) (end 153.911849 100.811849) (width 0.157) (layer F.Cu) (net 22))
 (segment (start 156.5 100.55) (end 156.146499 100.196499) (width 0.157) (layer F.Cu) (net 22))
 (segment (start 153.911849 102.464453) (end 153.472801 102.903501) (width 0.157) (layer F.Cu) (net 22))
 (segment (start 153.911849 100.811849) (end 153.911849 102.464453) (width 0.157) (layer F.Cu) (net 22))
 (segment (start 149.4 102.55) (end 149.5 102.45) (width 0.157) (layer F.Cu) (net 22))
 (segment (start 155.75 105.1807) (end 153.472801 102.903501) (width 0.157) (layer F.Cu) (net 22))
 (segment (start 155.75 106.75) (end 155.75 105.1807) (width 0.157) (layer F.Cu) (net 22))
 (segment (start 159.2 87.35) (end 159.05 87.2) (width 0.3) (layer B.Cu) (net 5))
 (segment (start 159.2 90.05) (end 159.2 87.35) (width 0.3) (layer B.Cu) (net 5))
 (segment (start 161.65 87.2) (end 154.15 87.2) (width 0.3) (layer B.Cu) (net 5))
 (segment (start 162 91) (end 164.5 91) (width 0.157) (layer F.Cu) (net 5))
 (segment (start 159.2 90.7) (end 159.5 91) (width 0.3) (layer B.Cu) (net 5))
 (segment (start 159.2 90.05) (end 159.2 90.7) (width 0.3) (layer B.Cu) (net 5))
 (segment (start 164.5 91) (end 159.5 91) (width 0.3) (layer B.Cu) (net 5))
 (segment (start 160.05 93.55) (end 160 93.55) (width 0.157) (layer F.Cu) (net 21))
 (segment (start 161 94.5) (end 160.05 93.55) (width 0.157) (layer F.Cu) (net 21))
 (segment (start 161 94.5) (end 161 98) (width 0.157) (layer F.Cu) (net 21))
 (segment (start 160.05 97.05) (end 160 97.05) (width 0.157) (layer F.Cu) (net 21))
 (segment (start 161 98) (end 160.05 97.05) (width 0.157) (layer F.Cu) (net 21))
 (segment (start 161 98) (end 161 101.5) (width 0.157) (layer F.Cu) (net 21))
 (segment (start 160.05 100.55) (end 160 100.55) (width 0.157) (layer F.Cu) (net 21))
 (segment (start 161 101.5) (end 160.05 100.55) (width 0.157) (layer F.Cu) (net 21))
 (segment (start 161 101.5) (end 161 105) (width 0.157) (layer F.Cu) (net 21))
 (segment (start 160.05 90.05) (end 160 90.05) (width 0.157) (layer F.Cu) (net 21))
 (segment (start 161 91) (end 160.05 90.05) (width 0.157) (layer F.Cu) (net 21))
 (segment (start 161 91) (end 161 94.5) (width 0.157) (layer F.Cu) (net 21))
 (segment (start 161 105) (end 161 106.75) (width 0.157) (layer F.Cu) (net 21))
 (segment (start 164.5 94.5) (end 162 94.5) (width 0.3) (layer F.Cu) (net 4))
 (segment (start 158.55 91.95) (end 158.55 90.05) (width 0.3) (layer B.Cu) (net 4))
 (segment (start 161.1 94.5) (end 158.55 91.95) (width 0.3) (layer B.Cu) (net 4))
 (segment (start 164.5 94.5) (end 161.1 94.5) (width 0.3) (layer B.Cu) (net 4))
 (segment (start 164.5 98) (end 162 98) (width 0.3) (layer F.Cu) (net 3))
 (segment (start 164.5 98) (end 161.4 98) (width 0.3) (layer B.Cu) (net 3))
 (segment (start 157.9 94.5) (end 157.9 93.1) (width 0.3) (layer B.Cu) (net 3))
 (segment (start 161.4 98) (end 157.9 94.5) (width 0.3) (layer B.Cu) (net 3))
 (segment (start 157.9 93.1) (end 157.9 90.05) (width 0.3) (layer B.Cu) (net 3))
 (segment (start 164.5 101.5) (end 162 101.5) (width 0.3) (layer F.Cu) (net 2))
 (segment (start 164.5 101.5) (end 161.2 101.5) (width 0.3) (layer B.Cu) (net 2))
 (segment (start 157.25 97.55) (end 157.25 90.05) (width 0.3) (layer B.Cu) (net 2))
 (segment (start 161.2 101.5) (end 157.25 97.55) (width 0.3) (layer B.Cu) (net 2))
 (segment (start 149.55 106.75) (end 149.4 106.9) (width 0.157) (layer F.Cu) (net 23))
 (segment (start 152.25 106.75) (end 149.55 106.75) (width 0.157) (layer F.Cu) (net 23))
 (segment (start 149.4 106.9) (end 145.4 106.9) (width 0.157) (layer F.Cu) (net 23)))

